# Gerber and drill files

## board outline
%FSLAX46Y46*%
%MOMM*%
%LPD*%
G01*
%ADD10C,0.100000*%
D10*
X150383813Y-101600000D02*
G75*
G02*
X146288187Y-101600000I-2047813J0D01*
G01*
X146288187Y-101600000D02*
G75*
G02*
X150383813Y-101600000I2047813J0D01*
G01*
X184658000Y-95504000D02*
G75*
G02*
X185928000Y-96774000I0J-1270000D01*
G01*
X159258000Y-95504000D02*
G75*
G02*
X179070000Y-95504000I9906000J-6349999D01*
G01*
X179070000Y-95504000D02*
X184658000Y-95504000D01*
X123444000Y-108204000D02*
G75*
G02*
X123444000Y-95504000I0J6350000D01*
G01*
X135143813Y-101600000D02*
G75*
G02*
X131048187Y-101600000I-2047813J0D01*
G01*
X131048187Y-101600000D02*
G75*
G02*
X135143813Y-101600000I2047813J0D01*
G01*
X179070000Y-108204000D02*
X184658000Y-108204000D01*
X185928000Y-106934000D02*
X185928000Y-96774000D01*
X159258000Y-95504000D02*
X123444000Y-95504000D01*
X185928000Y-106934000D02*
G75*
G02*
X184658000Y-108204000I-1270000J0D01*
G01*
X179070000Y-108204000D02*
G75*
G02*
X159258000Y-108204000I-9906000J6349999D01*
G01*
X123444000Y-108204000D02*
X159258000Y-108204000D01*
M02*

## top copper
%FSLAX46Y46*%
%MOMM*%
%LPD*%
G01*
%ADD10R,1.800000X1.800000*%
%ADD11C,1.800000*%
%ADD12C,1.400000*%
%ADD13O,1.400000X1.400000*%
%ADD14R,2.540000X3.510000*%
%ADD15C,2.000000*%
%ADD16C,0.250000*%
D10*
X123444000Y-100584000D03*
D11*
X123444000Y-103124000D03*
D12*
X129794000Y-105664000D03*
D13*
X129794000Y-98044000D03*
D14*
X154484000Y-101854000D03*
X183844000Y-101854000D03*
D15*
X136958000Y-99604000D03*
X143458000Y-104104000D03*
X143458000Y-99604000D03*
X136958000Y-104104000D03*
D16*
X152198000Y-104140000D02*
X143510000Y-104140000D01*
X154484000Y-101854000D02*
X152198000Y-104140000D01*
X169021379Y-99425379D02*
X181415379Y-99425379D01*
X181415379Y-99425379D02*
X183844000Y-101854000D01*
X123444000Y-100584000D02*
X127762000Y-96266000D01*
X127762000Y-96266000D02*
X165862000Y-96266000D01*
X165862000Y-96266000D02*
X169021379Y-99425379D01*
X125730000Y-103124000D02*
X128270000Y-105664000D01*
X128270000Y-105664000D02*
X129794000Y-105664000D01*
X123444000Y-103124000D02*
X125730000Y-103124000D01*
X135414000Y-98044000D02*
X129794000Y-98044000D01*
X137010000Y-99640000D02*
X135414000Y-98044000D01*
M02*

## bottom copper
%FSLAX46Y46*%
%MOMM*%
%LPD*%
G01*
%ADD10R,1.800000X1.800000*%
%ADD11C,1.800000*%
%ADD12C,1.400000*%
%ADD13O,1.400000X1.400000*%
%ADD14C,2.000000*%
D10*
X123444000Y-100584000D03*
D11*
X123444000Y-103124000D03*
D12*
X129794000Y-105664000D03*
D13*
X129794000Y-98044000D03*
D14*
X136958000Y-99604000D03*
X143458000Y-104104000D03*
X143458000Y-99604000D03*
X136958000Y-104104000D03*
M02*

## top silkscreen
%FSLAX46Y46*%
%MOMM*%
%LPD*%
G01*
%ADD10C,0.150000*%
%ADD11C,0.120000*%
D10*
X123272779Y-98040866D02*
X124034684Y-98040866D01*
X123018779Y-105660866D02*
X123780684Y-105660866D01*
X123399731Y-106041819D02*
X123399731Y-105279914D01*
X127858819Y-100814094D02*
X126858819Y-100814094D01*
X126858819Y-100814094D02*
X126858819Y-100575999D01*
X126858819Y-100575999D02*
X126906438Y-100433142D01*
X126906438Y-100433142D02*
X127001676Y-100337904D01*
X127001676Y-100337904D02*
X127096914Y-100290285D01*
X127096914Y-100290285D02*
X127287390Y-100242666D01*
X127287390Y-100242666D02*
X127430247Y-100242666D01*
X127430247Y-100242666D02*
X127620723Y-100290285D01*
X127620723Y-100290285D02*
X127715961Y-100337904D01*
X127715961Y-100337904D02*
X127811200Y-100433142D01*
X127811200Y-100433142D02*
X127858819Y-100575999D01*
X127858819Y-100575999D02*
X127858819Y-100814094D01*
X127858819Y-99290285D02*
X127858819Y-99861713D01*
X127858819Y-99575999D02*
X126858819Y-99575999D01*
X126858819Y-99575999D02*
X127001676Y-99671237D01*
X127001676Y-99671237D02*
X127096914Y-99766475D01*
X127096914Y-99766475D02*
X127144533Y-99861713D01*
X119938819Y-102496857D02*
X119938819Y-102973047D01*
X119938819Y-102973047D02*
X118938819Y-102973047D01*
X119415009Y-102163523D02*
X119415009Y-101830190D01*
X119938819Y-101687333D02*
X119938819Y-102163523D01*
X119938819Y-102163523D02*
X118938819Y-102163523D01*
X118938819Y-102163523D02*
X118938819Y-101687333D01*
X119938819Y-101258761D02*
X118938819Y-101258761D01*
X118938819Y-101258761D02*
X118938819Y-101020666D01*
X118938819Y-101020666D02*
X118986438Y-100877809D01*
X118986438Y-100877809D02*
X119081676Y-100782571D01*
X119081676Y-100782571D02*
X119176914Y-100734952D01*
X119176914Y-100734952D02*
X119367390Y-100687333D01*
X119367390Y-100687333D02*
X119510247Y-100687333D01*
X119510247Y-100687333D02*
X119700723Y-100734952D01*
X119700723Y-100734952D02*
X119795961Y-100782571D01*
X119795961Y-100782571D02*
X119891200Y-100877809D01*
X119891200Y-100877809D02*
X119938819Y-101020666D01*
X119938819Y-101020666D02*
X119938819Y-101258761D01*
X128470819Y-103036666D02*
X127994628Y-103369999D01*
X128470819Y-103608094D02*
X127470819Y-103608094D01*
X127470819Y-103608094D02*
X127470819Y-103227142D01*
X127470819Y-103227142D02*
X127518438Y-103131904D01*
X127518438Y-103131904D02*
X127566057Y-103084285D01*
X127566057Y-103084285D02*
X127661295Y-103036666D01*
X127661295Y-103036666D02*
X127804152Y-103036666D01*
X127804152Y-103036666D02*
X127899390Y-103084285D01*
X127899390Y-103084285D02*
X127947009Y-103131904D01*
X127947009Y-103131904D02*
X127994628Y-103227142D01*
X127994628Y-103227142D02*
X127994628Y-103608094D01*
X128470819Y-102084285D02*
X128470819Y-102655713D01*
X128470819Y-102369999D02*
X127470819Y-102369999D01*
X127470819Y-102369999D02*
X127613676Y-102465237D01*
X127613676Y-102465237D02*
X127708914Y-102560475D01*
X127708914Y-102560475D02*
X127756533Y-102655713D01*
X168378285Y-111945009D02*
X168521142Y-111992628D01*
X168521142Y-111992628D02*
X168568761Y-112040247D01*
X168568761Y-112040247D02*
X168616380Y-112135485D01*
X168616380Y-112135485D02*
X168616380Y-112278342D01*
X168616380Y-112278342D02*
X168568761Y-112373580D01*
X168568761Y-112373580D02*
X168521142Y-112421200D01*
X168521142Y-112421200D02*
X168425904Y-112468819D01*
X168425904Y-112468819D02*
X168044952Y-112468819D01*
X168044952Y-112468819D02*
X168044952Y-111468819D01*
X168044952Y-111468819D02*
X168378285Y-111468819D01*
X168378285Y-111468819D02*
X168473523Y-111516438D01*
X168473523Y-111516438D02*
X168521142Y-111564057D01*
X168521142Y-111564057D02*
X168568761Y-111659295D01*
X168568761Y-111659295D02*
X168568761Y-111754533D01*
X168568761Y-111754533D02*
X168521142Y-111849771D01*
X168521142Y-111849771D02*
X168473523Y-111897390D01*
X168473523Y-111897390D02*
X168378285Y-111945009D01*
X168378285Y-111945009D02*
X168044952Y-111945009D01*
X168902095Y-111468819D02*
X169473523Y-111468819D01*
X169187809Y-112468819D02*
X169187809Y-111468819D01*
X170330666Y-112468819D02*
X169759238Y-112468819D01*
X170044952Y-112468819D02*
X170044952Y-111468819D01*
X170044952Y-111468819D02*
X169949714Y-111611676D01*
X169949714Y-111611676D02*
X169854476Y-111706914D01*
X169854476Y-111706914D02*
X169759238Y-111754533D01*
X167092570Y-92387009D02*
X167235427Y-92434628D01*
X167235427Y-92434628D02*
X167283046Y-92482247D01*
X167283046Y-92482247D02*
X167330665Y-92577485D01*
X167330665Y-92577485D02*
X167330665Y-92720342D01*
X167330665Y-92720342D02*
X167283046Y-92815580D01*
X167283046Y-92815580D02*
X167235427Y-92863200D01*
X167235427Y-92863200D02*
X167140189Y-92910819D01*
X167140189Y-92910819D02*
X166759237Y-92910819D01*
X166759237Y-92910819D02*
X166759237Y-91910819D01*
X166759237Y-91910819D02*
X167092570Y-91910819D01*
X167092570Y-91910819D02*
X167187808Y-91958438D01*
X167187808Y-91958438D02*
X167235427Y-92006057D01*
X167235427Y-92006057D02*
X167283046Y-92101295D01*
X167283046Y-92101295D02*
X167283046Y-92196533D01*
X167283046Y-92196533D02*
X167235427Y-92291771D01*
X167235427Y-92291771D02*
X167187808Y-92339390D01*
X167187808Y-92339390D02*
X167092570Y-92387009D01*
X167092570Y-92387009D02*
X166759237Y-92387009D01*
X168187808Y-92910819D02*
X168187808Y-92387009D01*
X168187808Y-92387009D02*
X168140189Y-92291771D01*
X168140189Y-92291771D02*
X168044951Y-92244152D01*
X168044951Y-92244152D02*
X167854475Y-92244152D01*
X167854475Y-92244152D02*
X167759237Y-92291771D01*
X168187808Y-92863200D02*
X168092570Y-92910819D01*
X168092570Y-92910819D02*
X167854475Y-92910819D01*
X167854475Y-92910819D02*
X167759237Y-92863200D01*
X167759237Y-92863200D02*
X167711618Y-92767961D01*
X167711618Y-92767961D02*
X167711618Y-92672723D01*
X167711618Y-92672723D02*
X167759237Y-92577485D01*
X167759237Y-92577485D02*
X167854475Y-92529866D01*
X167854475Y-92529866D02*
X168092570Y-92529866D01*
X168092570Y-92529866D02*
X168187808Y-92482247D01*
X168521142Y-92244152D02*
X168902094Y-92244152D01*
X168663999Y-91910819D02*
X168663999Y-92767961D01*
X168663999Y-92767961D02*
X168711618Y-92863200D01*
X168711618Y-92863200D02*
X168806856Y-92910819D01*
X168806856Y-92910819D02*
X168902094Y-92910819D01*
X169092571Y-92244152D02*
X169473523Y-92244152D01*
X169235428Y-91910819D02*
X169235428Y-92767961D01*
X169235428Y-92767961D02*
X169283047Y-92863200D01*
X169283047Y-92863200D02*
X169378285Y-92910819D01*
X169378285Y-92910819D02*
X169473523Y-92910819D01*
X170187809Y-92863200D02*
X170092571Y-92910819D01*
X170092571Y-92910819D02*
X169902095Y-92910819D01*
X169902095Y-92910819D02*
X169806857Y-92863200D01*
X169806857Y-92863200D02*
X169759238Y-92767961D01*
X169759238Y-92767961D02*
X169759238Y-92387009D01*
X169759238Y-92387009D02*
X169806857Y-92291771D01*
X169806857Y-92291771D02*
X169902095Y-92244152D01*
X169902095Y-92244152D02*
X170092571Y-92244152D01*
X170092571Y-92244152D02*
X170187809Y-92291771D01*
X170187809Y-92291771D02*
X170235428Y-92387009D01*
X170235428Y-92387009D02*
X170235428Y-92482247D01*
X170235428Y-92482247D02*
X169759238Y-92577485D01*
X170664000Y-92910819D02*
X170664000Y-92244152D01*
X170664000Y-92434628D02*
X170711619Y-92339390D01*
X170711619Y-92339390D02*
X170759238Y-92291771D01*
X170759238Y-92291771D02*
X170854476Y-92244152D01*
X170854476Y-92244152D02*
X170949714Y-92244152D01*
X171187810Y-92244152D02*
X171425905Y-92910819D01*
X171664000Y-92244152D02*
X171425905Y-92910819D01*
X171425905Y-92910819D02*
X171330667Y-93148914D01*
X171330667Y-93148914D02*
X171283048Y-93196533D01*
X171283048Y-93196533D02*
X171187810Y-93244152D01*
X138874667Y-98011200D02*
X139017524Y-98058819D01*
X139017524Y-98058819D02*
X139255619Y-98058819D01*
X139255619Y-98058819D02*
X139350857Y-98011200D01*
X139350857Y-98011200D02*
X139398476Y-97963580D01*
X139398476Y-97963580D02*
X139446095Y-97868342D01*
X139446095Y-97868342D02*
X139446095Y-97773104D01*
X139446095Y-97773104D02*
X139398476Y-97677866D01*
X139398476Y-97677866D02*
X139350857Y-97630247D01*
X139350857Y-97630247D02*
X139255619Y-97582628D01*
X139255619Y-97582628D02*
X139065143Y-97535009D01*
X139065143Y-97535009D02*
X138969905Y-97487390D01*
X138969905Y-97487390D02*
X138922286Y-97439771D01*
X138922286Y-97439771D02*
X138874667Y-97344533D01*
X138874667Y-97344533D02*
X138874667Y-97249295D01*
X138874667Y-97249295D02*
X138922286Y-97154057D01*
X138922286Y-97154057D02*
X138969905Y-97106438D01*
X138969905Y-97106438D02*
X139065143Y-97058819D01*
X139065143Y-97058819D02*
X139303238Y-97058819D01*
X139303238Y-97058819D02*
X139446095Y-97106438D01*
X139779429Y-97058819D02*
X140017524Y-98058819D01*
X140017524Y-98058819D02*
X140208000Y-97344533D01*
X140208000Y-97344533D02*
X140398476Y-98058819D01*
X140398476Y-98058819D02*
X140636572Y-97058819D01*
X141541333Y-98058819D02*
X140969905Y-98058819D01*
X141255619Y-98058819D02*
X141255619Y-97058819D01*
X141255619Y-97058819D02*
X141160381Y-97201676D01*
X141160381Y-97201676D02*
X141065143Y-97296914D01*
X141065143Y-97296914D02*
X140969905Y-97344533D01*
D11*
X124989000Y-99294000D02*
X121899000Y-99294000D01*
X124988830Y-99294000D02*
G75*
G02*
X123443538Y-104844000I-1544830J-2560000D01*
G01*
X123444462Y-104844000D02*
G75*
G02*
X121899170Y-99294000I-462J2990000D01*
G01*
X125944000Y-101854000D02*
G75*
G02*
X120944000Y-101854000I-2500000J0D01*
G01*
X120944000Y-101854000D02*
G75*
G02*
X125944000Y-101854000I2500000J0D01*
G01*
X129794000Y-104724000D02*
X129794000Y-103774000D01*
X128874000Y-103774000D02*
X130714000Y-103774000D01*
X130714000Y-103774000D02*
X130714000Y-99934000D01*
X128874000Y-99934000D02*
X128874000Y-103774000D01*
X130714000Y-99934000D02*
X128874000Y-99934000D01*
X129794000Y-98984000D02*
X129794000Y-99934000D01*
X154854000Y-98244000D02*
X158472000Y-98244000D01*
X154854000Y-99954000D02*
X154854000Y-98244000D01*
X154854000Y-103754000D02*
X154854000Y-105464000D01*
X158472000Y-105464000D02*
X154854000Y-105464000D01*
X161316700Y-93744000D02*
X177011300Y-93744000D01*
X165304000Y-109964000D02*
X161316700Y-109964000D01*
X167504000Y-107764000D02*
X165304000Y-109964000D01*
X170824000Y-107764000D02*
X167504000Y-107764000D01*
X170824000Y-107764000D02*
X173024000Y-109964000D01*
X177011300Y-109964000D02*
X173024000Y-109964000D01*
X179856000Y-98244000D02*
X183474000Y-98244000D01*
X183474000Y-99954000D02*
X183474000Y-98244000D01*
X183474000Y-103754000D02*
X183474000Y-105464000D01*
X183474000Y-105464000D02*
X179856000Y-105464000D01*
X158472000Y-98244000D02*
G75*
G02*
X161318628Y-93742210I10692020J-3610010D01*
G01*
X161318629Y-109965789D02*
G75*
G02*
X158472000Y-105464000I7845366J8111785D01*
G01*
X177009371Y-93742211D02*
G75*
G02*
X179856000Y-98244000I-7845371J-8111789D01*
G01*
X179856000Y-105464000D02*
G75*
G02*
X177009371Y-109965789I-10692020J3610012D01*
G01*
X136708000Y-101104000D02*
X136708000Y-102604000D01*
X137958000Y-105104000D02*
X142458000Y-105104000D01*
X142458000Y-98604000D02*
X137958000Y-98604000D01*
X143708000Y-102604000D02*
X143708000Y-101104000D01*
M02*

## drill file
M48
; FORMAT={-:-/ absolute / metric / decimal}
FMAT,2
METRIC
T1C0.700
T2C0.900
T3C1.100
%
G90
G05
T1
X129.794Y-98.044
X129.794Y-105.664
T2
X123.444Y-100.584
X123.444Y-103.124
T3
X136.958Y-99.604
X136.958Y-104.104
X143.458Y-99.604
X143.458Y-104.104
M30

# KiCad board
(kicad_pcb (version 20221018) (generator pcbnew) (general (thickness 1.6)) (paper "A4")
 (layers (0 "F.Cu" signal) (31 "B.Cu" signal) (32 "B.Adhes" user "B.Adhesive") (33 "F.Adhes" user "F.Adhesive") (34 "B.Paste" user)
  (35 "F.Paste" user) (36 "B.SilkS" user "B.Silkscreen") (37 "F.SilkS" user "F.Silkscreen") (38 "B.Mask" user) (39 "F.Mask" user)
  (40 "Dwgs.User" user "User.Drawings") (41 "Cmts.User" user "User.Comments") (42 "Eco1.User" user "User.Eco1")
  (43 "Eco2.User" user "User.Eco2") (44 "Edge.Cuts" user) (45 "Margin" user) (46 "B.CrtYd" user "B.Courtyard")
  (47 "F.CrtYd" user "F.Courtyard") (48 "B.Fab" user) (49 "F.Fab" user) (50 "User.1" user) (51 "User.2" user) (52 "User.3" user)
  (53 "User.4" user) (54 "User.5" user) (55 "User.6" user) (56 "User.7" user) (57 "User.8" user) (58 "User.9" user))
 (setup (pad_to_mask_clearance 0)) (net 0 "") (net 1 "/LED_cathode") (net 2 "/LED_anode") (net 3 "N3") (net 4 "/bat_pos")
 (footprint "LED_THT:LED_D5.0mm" (layer "F.Cu") (at 123.444 100.584 -90)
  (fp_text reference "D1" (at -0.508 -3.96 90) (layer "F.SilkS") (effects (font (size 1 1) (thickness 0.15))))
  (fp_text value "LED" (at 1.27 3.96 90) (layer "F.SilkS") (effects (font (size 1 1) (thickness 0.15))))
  (fp_line (start -1.29 -1.545) (end -1.29 1.545) (stroke (width 0.12) (type solid)) (layer "F.SilkS"))
  (fp_arc (start -1.29 -1.54483) (mid 2.072002 -2.880433) (end 4.26 0.000462) (stroke (width 0.12) (type solid)) (layer "F.SilkS"))
  (fp_arc (start 4.26 -0.000462) (mid 2.072002 2.880433) (end -1.29 1.54483) (stroke (width 0.12) (type solid)) (layer "F.SilkS"))
  (fp_circle (center 1.27 0) (end 3.77 0) (stroke (width 0.12) (type solid)) (fill none) (layer "F.SilkS"))
  (pad "1" thru_hole rect (at 0 0 270) (size 1.8 1.8) (drill 0.9) (layers "*.Cu" "*.Mask") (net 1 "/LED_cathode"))
  (pad "2" thru_hole circle (at 2.54 0 270) (size 1.8 1.8) (drill 0.9) (layers "*.Cu" "*.Mask") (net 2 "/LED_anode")))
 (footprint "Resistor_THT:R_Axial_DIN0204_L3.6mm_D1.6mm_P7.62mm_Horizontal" (layer "F.Cu") (at 129.794 105.664 90)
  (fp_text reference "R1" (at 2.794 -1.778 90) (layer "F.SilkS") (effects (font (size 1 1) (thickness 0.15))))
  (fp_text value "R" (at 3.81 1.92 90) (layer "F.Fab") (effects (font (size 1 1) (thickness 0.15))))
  (fp_line (start 0.94 0) (end 1.89 0) (stroke (width 0.12) (type solid)) (layer "F.SilkS"))
  (fp_line (start 1.89 -0.92) (end 1.89 0.92) (stroke (width 0.12) (type solid)) (layer "F.SilkS"))
  (fp_line (start 1.89 0.92) (end 5.73 0.92) (stroke (width 0.12) (type solid)) (layer "F.SilkS"))
  (fp_line (start 5.73 -0.92) (end 1.89 -0.92) (stroke (width 0.12) (type solid)) (layer "F.SilkS"))
  (fp_line (start 5.73 0.92) (end 5.73 -0.92) (stroke (width 0.12) (type solid)) (layer "F.SilkS"))
  (fp_line (start 6.68 0) (end 5.73 0) (stroke (width 0.12) (type solid)) (layer "F.SilkS"))
  (pad "1" thru_hole circle (at 0 0 90) (size 1.4 1.4) (drill 0.7) (layers "*.Cu" "*.Mask") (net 2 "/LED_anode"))
  (pad "2" thru_hole oval (at 7.62 0 90) (size 1.4 1.4) (drill 0.7) (layers "*.Cu" "*.Mask") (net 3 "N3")))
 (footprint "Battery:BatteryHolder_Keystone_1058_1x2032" (layer "F.Cu") (at 169.164 101.854)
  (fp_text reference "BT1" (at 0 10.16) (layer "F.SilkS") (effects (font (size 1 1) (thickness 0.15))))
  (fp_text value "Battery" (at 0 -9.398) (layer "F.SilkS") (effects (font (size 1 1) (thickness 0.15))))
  (fp_line (start -14.31 -3.61) (end -10.692 -3.61) (stroke (width 0.12) (type solid)) (layer "F.SilkS"))
  (fp_line (start -14.31 -1.9) (end -14.31 -3.61) (stroke (width 0.12) (type solid)) (layer "F.SilkS"))
  (fp_line (start -14.31 1.9) (end -14.31 3.61) (stroke (width 0.12) (type solid)) (layer "F.SilkS"))
  (fp_line (start -10.692 3.61) (end -14.31 3.61) (stroke (width 0.12) (type solid)) (layer "F.SilkS"))
  (fp_line (start -7.8473 -8.11) (end 7.8473 -8.11) (stroke (width 0.12) (type solid)) (layer "F.SilkS"))
  (fp_line (start -3.86 8.11) (end -7.8473 8.11) (stroke (width 0.12) (type solid)) (layer "F.SilkS"))
  (fp_line (start -1.66 5.91) (end -3.86 8.11) (stroke (width 0.12) (type solid)) (layer "F.SilkS"))
  (fp_line (start 1.66 5.91) (end -1.66 5.91) (stroke (width 0.12) (type solid)) (layer "F.SilkS"))
  (fp_line (start 1.66 5.91) (end 3.86 8.11) (stroke (width 0.12) (type solid)) (layer "F.SilkS"))
  (fp_line (start 7.8473 8.11) (end 3.86 8.11) (stroke (width 0.12) (type solid)) (layer "F.SilkS"))
  (fp_line (start 10.692 -3.61) (end 14.31 -3.61) (stroke (width 0.12) (type solid)) (layer "F.SilkS"))
  (fp_line (start 14.31 -1.9) (end 14.31 -3.61) (stroke (width 0.12) (type solid)) (layer "F.SilkS"))
  (fp_line (start 14.31 1.9) (end 14.31 3.61) (stroke (width 0.12) (type solid)) (layer "F.SilkS"))
  (fp_line (start 14.31 3.61) (end 10.692 3.61) (stroke (width 0.12) (type solid)) (layer "F.SilkS"))
  (fp_arc (start -10.692 -3.61) (mid -9.538084 -6.031244) (end -7.845371 -8.111789) (stroke (width 0.12) (type solid)) (layer "F.SilkS"))
  (fp_arc (start -7.845371 8.111789) (mid -9.538085 6.031244) (end -10.692 3.61) (stroke (width 0.12) (type solid)) (layer "F.SilkS"))
  (fp_arc (start 7.845371 -8.111789) (mid 9.538085 -6.031244) (end 10.692 -3.61) (stroke (width 0.12) (type solid)) (layer "F.SilkS"))
  (fp_arc (start 10.692 3.61) (mid 9.538084 6.031244) (end 7.845371 8.111789) (stroke (width 0.12) (type solid)) (layer "F.SilkS"))
  (pad "1" smd rect (at -14.68 0) (size 2.54 3.51) (layers "F.Cu" "F.Paste" "F.Mask") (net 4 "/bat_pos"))
  (pad "2" smd rect (at 14.68 0) (size 2.54 3.51) (layers "F.Cu" "F.Paste" "F.Mask") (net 1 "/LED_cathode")))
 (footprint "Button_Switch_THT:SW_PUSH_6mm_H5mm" (layer "F.Cu") (at 136.958 99.604)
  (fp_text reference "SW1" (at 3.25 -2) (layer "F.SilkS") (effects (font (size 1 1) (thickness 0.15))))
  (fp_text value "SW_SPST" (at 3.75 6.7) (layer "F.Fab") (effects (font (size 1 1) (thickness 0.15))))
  (fp_line (start -0.25 1.5) (end -0.25 3) (stroke (width 0.12) (type solid)) (layer "F.SilkS"))
  (fp_line (start 1 5.5) (end 5.5 5.5) (stroke (width 0.12) (type solid)) (layer "F.SilkS"))
  (fp_line (start 5.5 -1) (end 1 -1) (stroke (width 0.12) (type solid)) (layer "F.SilkS"))
  (fp_line (start 6.75 3) (end 6.75 1.5) (stroke (width 0.12) (type solid)) (layer "F.SilkS"))
  (pad "1" thru_hole circle (at 0 0 90) (size 2 2) (drill 1.1) (layers "*.Cu" "*.Mask") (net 3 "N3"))
  (pad "2" thru_hole circle (at 6.5 4.5 90) (size 2 2) (drill 1.1) (layers "*.Cu" "*.Mask") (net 4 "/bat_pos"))
  (pad "3" thru_hole circle (at 6.5 0 90) (size 2 2) (drill 1.1) (layers "*.Cu" "*.Mask"))
  (pad "4" thru_hole circle (at 0 4.5 90) (size 2 2) (drill 1.1) (layers "*.Cu" "*.Mask")))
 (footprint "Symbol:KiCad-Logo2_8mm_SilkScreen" (layer "B.Cu") (at 169.164 101.854 180)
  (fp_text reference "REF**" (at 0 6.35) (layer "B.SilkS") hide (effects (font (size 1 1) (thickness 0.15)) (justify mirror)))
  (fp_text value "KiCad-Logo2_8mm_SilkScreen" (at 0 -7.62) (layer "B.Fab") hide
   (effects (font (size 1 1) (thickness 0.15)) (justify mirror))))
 (gr_circle (center 148.336 101.6) (end 150.114 102.616) (stroke (width 0.1) (type default)) (fill none) (layer "Edge.Cuts"))
 (gr_arc (start 184.658 95.504) (mid 185.556026 95.875974) (end 185.928 96.774) (stroke (width 0.1) (type default)) (layer "Edge.Cuts"))
 (gr_arc (start 159.258 95.504) (mid 169.164 90.087465) (end 179.07 95.504) (stroke (width 0.1) (type default)) (layer "Edge.Cuts"))
 (gr_line (start 179.07 95.504) (end 184.658 95.504) (stroke (width 0.1) (type default)) (layer "Edge.Cuts"))
 (gr_arc (start 123.444 108.204) (mid 117.094 101.854) (end 123.444 95.504) (stroke (width 0.1) (type default)) (layer "Edge.Cuts"))
 (gr_circle (center 133.096 101.6) (end 134.874 102.616) (stroke (width 0.1) (type default)) (fill none) (layer "Edge.Cuts"))
 (gr_line (start 179.07 108.204) (end 184.658 108.204) (stroke (width 0.1) (type default)) (layer "Edge.Cuts"))
 (gr_line (start 185.928 106.934) (end 185.928 96.774) (stroke (width 0.1) (type default)) (layer "Edge.Cuts"))
 (gr_line (start 159.258 95.504) (end 123.444 95.504) (stroke (width 0.1) (type default)) (layer "Edge.Cuts"))
 (gr_arc (start 185.928 106.934) (mid 185.556026 107.832026) (end 184.658 108.204) (stroke (width 0.1) (type default)) (layer "Edge.Cuts"))
 (gr_arc (start 179.07 108.204) (mid 169.164 113.620535) (end 159.258 108.204) (stroke (width 0.1) (type default)) (layer "Edge.Cuts"))
 (gr_line (start 123.444 108.204) (end 159.258 108.204) (stroke (width 0.1) (type default)) (layer "Edge.Cuts"))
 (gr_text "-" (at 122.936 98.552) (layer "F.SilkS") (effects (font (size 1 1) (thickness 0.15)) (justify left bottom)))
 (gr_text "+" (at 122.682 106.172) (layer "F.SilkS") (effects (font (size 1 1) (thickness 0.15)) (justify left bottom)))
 (segment (start 152.198 104.14) (end 143.51 104.14) (width 0.25) (layer "F.Cu") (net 4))
 (segment (start 154.484 101.854) (end 152.198 104.14) (width 0.25) (layer "F.Cu") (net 4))
 (segment (start 169.021379 99.425379) (end 181.415379 99.425379) (width 0.25) (layer "F.Cu") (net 1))
 (segment (start 181.415379 99.425379) (end 183.844 101.854) (width 0.25) (layer "F.Cu") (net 1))
 (segment (start 123.444 100.584) (end 127.762 96.266) (width 0.25) (layer "F.Cu") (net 1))
 (segment (start 127.762 96.266) (end 165.862 96.266) (width 0.25) (layer "F.Cu") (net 1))
 (segment (start 165.862 96.266) (end 169.021379 99.425379) (width 0.25) (layer "F.Cu") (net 1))
 (segment (start 125.73 103.124) (end 128.27 105.664) (width 0.25) (layer "F.Cu") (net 2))
 (segment (start 128.27 105.664) (end 129.794 105.664) (width 0.25) (layer "F.Cu") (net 2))
 (segment (start 123.444 103.124) (end 125.73 103.124) (width 0.25) (layer "F.Cu") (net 2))
 (segment (start 135.414 98.044) (end 129.794 98.044) (width 0.25) (layer "F.Cu") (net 3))
 (segment (start 137.01 99.64) (end 135.414 98.044) (width 0.25) (layer "F.Cu") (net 3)))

